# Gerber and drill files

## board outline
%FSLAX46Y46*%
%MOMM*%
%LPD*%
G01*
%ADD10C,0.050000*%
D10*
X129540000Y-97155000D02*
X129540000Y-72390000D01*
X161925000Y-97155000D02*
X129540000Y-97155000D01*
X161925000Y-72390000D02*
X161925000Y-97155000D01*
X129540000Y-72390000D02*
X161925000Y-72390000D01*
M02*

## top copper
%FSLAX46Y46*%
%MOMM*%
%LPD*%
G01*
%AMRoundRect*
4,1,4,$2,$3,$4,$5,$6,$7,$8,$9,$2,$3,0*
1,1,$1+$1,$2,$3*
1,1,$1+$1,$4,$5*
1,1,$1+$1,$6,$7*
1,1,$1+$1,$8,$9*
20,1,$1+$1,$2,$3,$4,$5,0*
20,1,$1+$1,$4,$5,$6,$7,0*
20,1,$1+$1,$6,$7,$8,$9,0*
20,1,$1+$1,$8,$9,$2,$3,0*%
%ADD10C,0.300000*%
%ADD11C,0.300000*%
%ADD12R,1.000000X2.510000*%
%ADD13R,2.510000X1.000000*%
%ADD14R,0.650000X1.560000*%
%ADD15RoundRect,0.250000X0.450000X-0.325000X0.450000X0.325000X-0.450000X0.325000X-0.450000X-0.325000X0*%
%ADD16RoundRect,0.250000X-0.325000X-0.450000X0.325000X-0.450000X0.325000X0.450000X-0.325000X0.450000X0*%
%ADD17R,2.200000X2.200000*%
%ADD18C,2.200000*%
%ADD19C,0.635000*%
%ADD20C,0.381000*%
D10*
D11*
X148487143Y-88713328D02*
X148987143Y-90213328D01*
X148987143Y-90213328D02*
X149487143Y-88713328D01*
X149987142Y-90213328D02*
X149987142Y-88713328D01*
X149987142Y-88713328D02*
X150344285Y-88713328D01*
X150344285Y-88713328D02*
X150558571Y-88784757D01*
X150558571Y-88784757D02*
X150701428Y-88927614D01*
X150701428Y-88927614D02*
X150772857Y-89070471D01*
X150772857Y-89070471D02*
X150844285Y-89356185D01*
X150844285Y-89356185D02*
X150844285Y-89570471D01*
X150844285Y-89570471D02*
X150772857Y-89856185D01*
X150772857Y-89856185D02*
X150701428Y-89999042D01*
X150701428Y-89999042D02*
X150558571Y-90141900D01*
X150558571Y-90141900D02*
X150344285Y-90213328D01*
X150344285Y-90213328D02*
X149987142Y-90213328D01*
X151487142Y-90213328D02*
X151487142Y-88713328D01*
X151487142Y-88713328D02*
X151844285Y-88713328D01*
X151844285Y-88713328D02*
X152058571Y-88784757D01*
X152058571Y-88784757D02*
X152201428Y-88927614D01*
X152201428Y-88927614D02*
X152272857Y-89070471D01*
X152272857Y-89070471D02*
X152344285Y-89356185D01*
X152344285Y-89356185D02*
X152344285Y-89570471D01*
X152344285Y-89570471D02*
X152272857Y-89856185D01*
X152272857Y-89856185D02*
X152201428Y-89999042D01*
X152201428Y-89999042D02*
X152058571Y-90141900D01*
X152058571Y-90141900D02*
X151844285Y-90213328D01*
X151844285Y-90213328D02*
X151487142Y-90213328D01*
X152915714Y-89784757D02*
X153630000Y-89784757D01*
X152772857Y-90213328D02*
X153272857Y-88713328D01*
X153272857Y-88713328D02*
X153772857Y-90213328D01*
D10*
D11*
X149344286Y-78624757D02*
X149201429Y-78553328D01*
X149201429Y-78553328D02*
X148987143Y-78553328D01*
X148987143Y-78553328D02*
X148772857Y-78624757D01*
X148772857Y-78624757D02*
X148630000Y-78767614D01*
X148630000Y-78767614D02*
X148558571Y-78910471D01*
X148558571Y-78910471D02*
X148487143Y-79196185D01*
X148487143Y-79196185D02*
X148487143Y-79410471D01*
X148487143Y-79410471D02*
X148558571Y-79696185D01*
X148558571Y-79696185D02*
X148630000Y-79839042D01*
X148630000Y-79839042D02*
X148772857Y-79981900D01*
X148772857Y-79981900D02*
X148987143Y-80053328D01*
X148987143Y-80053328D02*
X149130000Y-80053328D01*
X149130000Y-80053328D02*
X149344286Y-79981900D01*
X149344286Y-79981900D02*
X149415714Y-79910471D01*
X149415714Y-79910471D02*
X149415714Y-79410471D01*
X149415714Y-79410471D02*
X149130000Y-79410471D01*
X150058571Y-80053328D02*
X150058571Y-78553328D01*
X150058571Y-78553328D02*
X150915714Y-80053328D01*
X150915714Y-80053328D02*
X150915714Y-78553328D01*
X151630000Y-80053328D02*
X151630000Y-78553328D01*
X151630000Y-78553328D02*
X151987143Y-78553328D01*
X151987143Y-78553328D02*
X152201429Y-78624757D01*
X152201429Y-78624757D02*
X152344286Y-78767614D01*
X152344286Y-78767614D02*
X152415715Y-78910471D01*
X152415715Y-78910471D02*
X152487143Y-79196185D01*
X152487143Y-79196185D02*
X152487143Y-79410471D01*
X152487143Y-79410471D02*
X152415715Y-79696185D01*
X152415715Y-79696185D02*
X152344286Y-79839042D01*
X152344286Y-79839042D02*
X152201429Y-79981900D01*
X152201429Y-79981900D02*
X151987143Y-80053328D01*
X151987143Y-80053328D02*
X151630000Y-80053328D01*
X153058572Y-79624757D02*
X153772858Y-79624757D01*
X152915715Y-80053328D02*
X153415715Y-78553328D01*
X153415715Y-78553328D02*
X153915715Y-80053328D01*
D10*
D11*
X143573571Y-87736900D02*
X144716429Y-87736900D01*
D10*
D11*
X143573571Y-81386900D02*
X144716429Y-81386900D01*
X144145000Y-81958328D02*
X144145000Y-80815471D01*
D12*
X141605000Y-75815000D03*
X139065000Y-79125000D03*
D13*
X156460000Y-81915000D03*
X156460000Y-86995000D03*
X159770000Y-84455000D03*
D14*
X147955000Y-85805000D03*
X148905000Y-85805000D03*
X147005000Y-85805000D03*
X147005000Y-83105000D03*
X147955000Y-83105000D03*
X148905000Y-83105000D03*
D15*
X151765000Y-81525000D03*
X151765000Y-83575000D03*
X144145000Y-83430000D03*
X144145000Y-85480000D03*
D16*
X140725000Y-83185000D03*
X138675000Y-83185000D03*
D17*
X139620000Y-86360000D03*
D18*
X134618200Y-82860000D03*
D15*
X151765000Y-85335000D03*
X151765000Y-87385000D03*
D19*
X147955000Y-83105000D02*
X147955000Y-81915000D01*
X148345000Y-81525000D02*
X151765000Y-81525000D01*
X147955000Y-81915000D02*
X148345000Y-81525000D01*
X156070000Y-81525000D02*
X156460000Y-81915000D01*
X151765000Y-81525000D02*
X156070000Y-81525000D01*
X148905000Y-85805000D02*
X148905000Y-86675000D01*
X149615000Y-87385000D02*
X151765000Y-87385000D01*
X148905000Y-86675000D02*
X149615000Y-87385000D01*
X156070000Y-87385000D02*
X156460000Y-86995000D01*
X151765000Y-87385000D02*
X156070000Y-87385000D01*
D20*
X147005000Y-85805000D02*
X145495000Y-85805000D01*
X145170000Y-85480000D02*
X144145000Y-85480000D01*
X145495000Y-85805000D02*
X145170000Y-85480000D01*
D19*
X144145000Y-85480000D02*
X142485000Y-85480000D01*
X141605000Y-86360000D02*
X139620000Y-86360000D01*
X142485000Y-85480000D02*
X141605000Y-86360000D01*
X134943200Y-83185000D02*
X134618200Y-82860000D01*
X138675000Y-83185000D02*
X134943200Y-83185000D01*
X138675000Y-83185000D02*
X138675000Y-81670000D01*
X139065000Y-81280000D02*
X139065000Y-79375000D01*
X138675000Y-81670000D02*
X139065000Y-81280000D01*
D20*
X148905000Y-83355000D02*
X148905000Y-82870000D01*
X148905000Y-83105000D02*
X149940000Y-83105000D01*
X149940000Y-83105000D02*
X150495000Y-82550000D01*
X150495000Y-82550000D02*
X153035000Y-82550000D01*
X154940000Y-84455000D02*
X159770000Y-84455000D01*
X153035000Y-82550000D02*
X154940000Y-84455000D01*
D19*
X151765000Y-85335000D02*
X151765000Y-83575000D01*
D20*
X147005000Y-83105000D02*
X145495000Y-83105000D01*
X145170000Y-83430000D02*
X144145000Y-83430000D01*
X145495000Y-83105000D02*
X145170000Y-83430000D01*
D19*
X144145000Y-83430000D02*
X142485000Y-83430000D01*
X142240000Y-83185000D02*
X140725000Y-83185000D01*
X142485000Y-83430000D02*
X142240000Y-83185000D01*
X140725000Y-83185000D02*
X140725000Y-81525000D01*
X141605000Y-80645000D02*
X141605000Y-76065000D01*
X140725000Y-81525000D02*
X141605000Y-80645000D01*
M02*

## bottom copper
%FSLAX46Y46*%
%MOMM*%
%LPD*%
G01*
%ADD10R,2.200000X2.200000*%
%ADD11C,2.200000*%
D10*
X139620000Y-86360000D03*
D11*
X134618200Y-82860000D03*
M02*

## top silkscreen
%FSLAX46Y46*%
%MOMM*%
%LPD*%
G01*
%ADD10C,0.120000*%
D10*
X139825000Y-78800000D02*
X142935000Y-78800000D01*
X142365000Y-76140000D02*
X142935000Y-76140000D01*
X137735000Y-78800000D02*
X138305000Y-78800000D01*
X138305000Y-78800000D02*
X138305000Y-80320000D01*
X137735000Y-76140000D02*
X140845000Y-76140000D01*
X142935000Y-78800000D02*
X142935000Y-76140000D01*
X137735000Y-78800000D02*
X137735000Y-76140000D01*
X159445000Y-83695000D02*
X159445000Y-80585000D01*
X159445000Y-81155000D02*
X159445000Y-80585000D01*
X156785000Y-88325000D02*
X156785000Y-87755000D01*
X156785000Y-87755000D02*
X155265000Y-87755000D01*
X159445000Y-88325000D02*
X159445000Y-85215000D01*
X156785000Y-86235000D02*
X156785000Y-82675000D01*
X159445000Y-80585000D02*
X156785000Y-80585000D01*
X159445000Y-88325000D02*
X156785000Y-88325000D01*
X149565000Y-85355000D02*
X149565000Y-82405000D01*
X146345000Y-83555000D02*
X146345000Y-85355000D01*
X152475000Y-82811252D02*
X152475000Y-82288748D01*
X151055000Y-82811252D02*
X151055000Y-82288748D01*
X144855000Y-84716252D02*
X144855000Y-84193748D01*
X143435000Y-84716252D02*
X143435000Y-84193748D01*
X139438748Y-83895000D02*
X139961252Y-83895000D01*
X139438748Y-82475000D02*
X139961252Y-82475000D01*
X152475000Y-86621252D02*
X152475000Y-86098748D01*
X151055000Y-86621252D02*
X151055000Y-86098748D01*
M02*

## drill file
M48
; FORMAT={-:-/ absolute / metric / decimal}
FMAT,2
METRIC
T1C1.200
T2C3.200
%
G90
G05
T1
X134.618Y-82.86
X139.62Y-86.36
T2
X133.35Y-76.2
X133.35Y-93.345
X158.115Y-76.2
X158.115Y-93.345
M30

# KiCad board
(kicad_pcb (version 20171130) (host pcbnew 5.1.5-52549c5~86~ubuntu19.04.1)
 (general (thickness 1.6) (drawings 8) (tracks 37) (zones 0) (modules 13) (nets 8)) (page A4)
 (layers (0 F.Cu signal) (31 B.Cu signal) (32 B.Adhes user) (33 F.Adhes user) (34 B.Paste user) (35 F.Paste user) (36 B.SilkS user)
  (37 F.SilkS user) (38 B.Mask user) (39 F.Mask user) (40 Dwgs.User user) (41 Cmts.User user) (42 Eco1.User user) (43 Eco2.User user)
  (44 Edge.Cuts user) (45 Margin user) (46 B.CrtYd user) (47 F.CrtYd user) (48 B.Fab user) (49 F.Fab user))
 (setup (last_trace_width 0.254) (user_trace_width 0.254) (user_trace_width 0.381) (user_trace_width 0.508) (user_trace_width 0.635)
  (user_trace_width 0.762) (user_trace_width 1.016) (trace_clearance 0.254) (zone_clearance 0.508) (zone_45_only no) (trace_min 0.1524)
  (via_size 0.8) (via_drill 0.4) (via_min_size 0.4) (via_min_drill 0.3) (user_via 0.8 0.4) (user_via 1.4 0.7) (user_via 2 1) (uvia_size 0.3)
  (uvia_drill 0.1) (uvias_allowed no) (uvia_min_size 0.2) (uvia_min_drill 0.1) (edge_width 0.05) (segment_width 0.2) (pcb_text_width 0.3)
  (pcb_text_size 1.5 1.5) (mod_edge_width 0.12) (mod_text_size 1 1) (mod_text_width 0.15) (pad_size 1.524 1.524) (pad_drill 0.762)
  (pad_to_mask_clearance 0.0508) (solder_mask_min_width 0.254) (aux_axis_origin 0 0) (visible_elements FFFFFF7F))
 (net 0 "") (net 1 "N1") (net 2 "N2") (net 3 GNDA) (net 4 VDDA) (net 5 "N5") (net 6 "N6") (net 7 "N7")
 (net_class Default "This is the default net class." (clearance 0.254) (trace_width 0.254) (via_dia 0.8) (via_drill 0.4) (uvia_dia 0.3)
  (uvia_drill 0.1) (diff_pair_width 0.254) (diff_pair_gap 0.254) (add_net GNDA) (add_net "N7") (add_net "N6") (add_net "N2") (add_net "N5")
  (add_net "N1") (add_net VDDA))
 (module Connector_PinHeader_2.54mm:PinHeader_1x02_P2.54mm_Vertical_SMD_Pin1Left (layer F.Cu) (at 140.335 77.47 90)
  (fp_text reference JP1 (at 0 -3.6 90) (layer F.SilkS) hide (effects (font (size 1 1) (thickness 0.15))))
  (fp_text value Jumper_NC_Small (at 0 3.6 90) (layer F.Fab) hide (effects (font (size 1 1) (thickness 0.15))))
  (fp_line (start -1.33 -0.51) (end -1.33 2.6) (layer F.SilkS) (width 0.12))
  (fp_line (start 1.33 2.03) (end 1.33 2.6) (layer F.SilkS) (width 0.12))
  (fp_line (start -1.33 -2.6) (end -1.33 -2.03) (layer F.SilkS) (width 0.12))
  (fp_line (start -1.33 -2.03) (end -2.85 -2.03) (layer F.SilkS) (width 0.12))
  (fp_line (start 1.33 -2.6) (end 1.33 0.51) (layer F.SilkS) (width 0.12))
  (fp_line (start -1.33 2.6) (end 1.33 2.6) (layer F.SilkS) (width 0.12))
  (fp_line (start -1.33 -2.6) (end 1.33 -2.6) (layer F.SilkS) (width 0.12))
  (pad 2 smd rect (at 1.655 1.27 90) (size 2.51 1) (layers F.Cu F.Paste F.Mask) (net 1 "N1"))
  (pad 1 smd rect (at -1.655 -1.27 90) (size 2.51 1) (layers F.Cu F.Paste F.Mask) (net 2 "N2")))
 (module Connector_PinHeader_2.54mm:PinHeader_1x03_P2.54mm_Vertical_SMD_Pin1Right (layer F.Cu) (at 158.115 84.455 180)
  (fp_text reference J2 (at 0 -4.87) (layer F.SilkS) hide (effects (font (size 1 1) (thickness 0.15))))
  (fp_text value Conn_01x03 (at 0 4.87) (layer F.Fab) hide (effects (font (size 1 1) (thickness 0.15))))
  (fp_line (start -1.33 0.76) (end -1.33 3.87) (layer F.SilkS) (width 0.12))
  (fp_line (start -1.33 3.3) (end -1.33 3.87) (layer F.SilkS) (width 0.12))
  (fp_line (start 1.33 -3.87) (end 1.33 -3.3) (layer F.SilkS) (width 0.12))
  (fp_line (start 1.33 -3.3) (end 2.85 -3.3) (layer F.SilkS) (width 0.12))
  (fp_line (start -1.33 -3.87) (end -1.33 -0.76) (layer F.SilkS) (width 0.12))
  (fp_line (start 1.33 -1.78) (end 1.33 1.78) (layer F.SilkS) (width 0.12))
  (fp_line (start -1.33 3.87) (end 1.33 3.87) (layer F.SilkS) (width 0.12))
  (fp_line (start -1.33 -3.87) (end 1.33 -3.87) (layer F.SilkS) (width 0.12))
  (pad 3 smd rect (at 1.655 2.54 180) (size 2.51 1) (layers F.Cu F.Paste F.Mask) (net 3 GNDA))
  (pad 1 smd rect (at 1.655 -2.54 180) (size 2.51 1) (layers F.Cu F.Paste F.Mask) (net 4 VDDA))
  (pad 2 smd rect (at -1.655 0 180) (size 2.51 1) (layers F.Cu F.Paste F.Mask) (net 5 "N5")))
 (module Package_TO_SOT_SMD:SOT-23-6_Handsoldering (layer F.Cu) (at 147.955 84.455 270)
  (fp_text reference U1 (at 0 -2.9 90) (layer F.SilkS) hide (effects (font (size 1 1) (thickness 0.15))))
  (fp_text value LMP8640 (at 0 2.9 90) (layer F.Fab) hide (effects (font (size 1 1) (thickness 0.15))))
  (fp_line (start 0.9 -1.61) (end -2.05 -1.61) (layer F.SilkS) (width 0.12))
  (fp_line (start -0.9 1.61) (end 0.9 1.61) (layer F.SilkS) (width 0.12))
  (pad 5 smd rect (at 1.35 0 270) (size 1.56 0.65) (layers F.Cu F.Paste F.Mask))
  (pad 6 smd rect (at 1.35 -0.95 270) (size 1.56 0.65) (layers F.Cu F.Paste F.Mask) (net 4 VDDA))
  (pad 4 smd rect (at 1.35 0.95 270) (size 1.56 0.65) (layers F.Cu F.Paste F.Mask) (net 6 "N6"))
  (pad 3 smd rect (at -1.35 0.95 270) (size 1.56 0.65) (layers F.Cu F.Paste F.Mask) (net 1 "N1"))
  (pad 2 smd rect (at -1.35 0 270) (size 1.56 0.65) (layers F.Cu F.Paste F.Mask) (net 3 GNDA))
  (pad 1 smd rect (at -1.35 -0.95 270) (size 1.56 0.65) (layers F.Cu F.Paste F.Mask) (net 5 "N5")))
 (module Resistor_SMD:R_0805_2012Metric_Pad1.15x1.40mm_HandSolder (layer F.Cu) (at 151.765 82.55 90)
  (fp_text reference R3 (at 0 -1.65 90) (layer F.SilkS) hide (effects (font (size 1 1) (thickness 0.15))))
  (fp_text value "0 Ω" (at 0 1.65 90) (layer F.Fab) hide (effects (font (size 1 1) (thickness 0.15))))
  (fp_line (start -0.261252 0.71) (end 0.261252 0.71) (layer F.SilkS) (width 0.12))
  (fp_line (start -0.261252 -0.71) (end 0.261252 -0.71) (layer F.SilkS) (width 0.12))
  (pad 2 smd roundrect (at 1.025 0 90) (size 1.15 1.4) (layers F.Cu F.Paste F.Mask) (roundrect_rratio 0.217391) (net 3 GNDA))
  (pad 1 smd roundrect (at -1.025 0 90) (size 1.15 1.4) (layers F.Cu F.Paste F.Mask) (roundrect_rratio 0.217391) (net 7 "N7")))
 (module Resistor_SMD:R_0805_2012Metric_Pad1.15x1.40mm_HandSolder (layer F.Cu) (at 144.145 84.455 90)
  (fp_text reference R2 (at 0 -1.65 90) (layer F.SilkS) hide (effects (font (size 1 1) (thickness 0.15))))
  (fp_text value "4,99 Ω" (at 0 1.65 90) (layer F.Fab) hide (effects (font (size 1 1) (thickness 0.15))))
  (fp_line (start -0.261252 0.71) (end 0.261252 0.71) (layer F.SilkS) (width 0.12))
  (fp_line (start -0.261252 -0.71) (end 0.261252 -0.71) (layer F.SilkS) (width 0.12))
  (pad 2 smd roundrect (at 1.025 0 90) (size 1.15 1.4) (layers F.Cu F.Paste F.Mask) (roundrect_rratio 0.217391) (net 1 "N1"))
  (pad 1 smd roundrect (at -1.025 0 90) (size 1.15 1.4) (layers F.Cu F.Paste F.Mask) (roundrect_rratio 0.217391) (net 6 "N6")))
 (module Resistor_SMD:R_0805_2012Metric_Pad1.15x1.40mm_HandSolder (layer F.Cu) (at 139.7 83.185)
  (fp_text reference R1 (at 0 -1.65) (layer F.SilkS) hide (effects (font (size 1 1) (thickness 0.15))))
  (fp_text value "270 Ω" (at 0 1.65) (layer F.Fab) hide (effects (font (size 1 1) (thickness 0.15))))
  (fp_line (start -0.261252 0.71) (end 0.261252 0.71) (layer F.SilkS) (width 0.12))
  (fp_line (start -0.261252 -0.71) (end 0.261252 -0.71) (layer F.SilkS) (width 0.12))
  (pad 2 smd roundrect (at 1.025 0) (size 1.15 1.4) (layers F.Cu F.Paste F.Mask) (roundrect_rratio 0.217391) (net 1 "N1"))
  (pad 1 smd roundrect (at -1.025 0) (size 1.15 1.4) (layers F.Cu F.Paste F.Mask) (roundrect_rratio 0.217391) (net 2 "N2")))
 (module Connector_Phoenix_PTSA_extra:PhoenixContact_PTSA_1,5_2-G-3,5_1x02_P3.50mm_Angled (layer B.Cu) (at 134.62 86.36 90)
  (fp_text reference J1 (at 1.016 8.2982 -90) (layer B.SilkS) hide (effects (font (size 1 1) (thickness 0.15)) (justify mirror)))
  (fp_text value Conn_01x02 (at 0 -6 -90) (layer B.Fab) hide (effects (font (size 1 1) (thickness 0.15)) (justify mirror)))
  (pad 1 thru_hole rect (at 0 5 90) (size 2.2 2.2) (drill 1.2) (layers *.Cu *.Mask) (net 6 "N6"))
  (pad 2 thru_hole circle (at 3.5 -0.0018 90) (size 2.2 2.2) (drill 1.2) (layers *.Cu *.Mask) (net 2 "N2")))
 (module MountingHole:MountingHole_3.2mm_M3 (layer F.Cu) (at 133.35 93.345)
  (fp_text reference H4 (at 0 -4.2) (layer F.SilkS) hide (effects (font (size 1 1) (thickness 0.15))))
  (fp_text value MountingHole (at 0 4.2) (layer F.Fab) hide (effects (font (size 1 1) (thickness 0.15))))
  (pad 1 np_thru_hole circle (at 0 0) (size 3.2 3.2) (drill 3.2) (layers *.Cu *.Mask)))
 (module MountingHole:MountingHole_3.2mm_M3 (layer F.Cu) (at 158.115 93.345)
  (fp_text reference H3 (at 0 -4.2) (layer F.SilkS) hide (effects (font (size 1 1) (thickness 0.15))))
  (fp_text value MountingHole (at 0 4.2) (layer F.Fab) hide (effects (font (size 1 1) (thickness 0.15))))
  (pad 1 np_thru_hole circle (at 0 0) (size 3.2 3.2) (drill 3.2) (layers *.Cu *.Mask)))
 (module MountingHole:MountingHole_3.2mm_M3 (layer F.Cu) (at 158.115 76.2)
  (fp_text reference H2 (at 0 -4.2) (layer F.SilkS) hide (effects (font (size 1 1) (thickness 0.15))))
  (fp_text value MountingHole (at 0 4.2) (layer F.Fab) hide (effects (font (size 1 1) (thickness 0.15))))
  (pad 1 np_thru_hole circle (at 0 0) (size 3.2 3.2) (drill 3.2) (layers *.Cu *.Mask)))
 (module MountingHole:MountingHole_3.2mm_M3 (layer F.Cu) (at 133.35 76.2)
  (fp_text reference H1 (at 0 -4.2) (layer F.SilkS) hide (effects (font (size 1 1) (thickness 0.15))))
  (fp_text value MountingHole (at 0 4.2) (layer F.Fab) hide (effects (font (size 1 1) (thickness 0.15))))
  (pad 1 np_thru_hole circle (at 0 0) (size 3.2 3.2) (drill 3.2) (layers *.Cu *.Mask)))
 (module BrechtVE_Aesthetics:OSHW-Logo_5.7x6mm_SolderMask (layer F.Cu) (at 145.415 92.71)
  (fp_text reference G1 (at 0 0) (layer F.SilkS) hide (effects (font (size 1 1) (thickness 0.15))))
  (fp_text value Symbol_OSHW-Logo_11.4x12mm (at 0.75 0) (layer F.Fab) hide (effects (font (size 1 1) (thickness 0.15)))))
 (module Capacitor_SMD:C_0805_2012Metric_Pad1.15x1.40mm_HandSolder (layer F.Cu) (at 151.765 86.36 90)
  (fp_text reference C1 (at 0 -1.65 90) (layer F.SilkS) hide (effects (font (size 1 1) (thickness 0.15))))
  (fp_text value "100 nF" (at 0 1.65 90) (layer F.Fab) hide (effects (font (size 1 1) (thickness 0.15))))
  (fp_line (start -0.261252 0.71) (end 0.261252 0.71) (layer F.SilkS) (width 0.12))
  (fp_line (start -0.261252 -0.71) (end 0.261252 -0.71) (layer F.SilkS) (width 0.12))
  (pad 2 smd roundrect (at 1.025 0 90) (size 1.15 1.4) (layers F.Cu F.Paste F.Mask) (roundrect_rratio 0.217391) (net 7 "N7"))
  (pad 1 smd roundrect (at -1.025 0 90) (size 1.15 1.4) (layers F.Cu F.Paste F.Mask) (roundrect_rratio 0.217391) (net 4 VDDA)))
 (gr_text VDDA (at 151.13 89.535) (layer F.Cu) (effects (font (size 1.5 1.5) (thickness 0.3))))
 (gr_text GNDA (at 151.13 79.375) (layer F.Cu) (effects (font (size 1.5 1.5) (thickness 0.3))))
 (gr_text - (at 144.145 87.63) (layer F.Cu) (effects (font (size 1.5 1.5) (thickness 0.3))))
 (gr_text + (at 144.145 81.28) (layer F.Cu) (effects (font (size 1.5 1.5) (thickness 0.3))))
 (gr_line (start 129.54 97.155) (end 129.54 72.39) (layer Edge.Cuts) (width 0.05))
 (gr_line (start 161.925 97.155) (end 129.54 97.155) (layer Edge.Cuts) (width 0.05))
 (gr_line (start 161.925 72.39) (end 161.925 97.155) (layer Edge.Cuts) (width 0.05))
 (gr_line (start 129.54 72.39) (end 161.925 72.39) (layer Edge.Cuts) (width 0.05))
 (segment (start 147.955 83.105) (end 147.955 81.915) (width 0.635) (layer F.Cu) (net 3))
 (segment (start 148.345 81.525) (end 151.765 81.525) (width 0.635) (layer F.Cu) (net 3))
 (segment (start 147.955 81.915) (end 148.345 81.525) (width 0.635) (layer F.Cu) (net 3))
 (segment (start 156.07 81.525) (end 156.46 81.915) (width 0.635) (layer F.Cu) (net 3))
 (segment (start 151.765 81.525) (end 156.07 81.525) (width 0.635) (layer F.Cu) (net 3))
 (segment (start 148.905 85.805) (end 148.905 86.675) (width 0.635) (layer F.Cu) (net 4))
 (segment (start 149.615 87.385) (end 151.765 87.385) (width 0.635) (layer F.Cu) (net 4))
 (segment (start 148.905 86.675) (end 149.615 87.385) (width 0.635) (layer F.Cu) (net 4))
 (segment (start 156.07 87.385) (end 156.46 86.995) (width 0.635) (layer F.Cu) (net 4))
 (segment (start 151.765 87.385) (end 156.07 87.385) (width 0.635) (layer F.Cu) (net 4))
 (segment (start 147.005 85.805) (end 145.495 85.805) (width 0.381) (layer F.Cu) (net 6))
 (segment (start 145.17 85.48) (end 144.145 85.48) (width 0.381) (layer F.Cu) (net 6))
 (segment (start 145.495 85.805) (end 145.17 85.48) (width 0.381) (layer F.Cu) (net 6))
 (segment (start 144.145 85.48) (end 142.485 85.48) (width 0.635) (layer F.Cu) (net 6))
 (segment (start 141.605 86.36) (end 139.62 86.36) (width 0.635) (layer F.Cu) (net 6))
 (segment (start 142.485 85.48) (end 141.605 86.36) (width 0.635) (layer F.Cu) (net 6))
 (segment (start 134.9432 83.185) (end 134.6182 82.86) (width 0.635) (layer F.Cu) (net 2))
 (segment (start 138.675 83.185) (end 134.9432 83.185) (width 0.635) (layer F.Cu) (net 2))
 (segment (start 138.675 83.185) (end 138.675 81.67) (width 0.635) (layer F.Cu) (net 2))
 (segment (start 139.065 81.28) (end 139.065 79.375) (width 0.635) (layer F.Cu) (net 2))
 (segment (start 138.675 81.67) (end 139.065 81.28) (width 0.635) (layer F.Cu) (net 2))
 (segment (start 148.905 83.355) (end 148.905 82.87) (width 0.381) (layer F.Cu) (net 5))
 (segment (start 148.905 83.105) (end 149.94 83.105) (width 0.381) (layer F.Cu) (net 5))
 (segment (start 149.94 83.105) (end 150.495 82.55) (width 0.381) (layer F.Cu) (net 5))
 (segment (start 150.495 82.55) (end 153.035 82.55) (width 0.381) (layer F.Cu) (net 5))
 (segment (start 154.94 84.455) (end 159.77 84.455) (width 0.381) (layer F.Cu) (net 5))
 (segment (start 153.035 82.55) (end 154.94 84.455) (width 0.381) (layer F.Cu) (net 5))
 (segment (start 151.765 85.335) (end 151.765 83.575) (width 0.635) (layer F.Cu) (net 7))
 (segment (start 147.005 83.105) (end 145.495 83.105) (width 0.381) (layer F.Cu) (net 1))
 (segment (start 145.17 83.43) (end 144.145 83.43) (width 0.381) (layer F.Cu) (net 1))
 (segment (start 145.495 83.105) (end 145.17 83.43) (width 0.381) (layer F.Cu) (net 1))
 (segment (start 144.145 83.43) (end 142.485 83.43) (width 0.635) (layer F.Cu) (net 1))
 (segment (start 142.24 83.185) (end 140.725 83.185) (width 0.635) (layer F.Cu) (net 1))
 (segment (start 142.485 83.43) (end 142.24 83.185) (width 0.635) (layer F.Cu) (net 1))
 (segment (start 140.725 83.185) (end 140.725 81.525) (width 0.635) (layer F.Cu) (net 1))
 (segment (start 141.605 80.645) (end 141.605 76.065) (width 0.635) (layer F.Cu) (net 1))
 (segment (start 140.725 81.525) (end 141.605 80.645) (width 0.635) (layer F.Cu) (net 1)))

